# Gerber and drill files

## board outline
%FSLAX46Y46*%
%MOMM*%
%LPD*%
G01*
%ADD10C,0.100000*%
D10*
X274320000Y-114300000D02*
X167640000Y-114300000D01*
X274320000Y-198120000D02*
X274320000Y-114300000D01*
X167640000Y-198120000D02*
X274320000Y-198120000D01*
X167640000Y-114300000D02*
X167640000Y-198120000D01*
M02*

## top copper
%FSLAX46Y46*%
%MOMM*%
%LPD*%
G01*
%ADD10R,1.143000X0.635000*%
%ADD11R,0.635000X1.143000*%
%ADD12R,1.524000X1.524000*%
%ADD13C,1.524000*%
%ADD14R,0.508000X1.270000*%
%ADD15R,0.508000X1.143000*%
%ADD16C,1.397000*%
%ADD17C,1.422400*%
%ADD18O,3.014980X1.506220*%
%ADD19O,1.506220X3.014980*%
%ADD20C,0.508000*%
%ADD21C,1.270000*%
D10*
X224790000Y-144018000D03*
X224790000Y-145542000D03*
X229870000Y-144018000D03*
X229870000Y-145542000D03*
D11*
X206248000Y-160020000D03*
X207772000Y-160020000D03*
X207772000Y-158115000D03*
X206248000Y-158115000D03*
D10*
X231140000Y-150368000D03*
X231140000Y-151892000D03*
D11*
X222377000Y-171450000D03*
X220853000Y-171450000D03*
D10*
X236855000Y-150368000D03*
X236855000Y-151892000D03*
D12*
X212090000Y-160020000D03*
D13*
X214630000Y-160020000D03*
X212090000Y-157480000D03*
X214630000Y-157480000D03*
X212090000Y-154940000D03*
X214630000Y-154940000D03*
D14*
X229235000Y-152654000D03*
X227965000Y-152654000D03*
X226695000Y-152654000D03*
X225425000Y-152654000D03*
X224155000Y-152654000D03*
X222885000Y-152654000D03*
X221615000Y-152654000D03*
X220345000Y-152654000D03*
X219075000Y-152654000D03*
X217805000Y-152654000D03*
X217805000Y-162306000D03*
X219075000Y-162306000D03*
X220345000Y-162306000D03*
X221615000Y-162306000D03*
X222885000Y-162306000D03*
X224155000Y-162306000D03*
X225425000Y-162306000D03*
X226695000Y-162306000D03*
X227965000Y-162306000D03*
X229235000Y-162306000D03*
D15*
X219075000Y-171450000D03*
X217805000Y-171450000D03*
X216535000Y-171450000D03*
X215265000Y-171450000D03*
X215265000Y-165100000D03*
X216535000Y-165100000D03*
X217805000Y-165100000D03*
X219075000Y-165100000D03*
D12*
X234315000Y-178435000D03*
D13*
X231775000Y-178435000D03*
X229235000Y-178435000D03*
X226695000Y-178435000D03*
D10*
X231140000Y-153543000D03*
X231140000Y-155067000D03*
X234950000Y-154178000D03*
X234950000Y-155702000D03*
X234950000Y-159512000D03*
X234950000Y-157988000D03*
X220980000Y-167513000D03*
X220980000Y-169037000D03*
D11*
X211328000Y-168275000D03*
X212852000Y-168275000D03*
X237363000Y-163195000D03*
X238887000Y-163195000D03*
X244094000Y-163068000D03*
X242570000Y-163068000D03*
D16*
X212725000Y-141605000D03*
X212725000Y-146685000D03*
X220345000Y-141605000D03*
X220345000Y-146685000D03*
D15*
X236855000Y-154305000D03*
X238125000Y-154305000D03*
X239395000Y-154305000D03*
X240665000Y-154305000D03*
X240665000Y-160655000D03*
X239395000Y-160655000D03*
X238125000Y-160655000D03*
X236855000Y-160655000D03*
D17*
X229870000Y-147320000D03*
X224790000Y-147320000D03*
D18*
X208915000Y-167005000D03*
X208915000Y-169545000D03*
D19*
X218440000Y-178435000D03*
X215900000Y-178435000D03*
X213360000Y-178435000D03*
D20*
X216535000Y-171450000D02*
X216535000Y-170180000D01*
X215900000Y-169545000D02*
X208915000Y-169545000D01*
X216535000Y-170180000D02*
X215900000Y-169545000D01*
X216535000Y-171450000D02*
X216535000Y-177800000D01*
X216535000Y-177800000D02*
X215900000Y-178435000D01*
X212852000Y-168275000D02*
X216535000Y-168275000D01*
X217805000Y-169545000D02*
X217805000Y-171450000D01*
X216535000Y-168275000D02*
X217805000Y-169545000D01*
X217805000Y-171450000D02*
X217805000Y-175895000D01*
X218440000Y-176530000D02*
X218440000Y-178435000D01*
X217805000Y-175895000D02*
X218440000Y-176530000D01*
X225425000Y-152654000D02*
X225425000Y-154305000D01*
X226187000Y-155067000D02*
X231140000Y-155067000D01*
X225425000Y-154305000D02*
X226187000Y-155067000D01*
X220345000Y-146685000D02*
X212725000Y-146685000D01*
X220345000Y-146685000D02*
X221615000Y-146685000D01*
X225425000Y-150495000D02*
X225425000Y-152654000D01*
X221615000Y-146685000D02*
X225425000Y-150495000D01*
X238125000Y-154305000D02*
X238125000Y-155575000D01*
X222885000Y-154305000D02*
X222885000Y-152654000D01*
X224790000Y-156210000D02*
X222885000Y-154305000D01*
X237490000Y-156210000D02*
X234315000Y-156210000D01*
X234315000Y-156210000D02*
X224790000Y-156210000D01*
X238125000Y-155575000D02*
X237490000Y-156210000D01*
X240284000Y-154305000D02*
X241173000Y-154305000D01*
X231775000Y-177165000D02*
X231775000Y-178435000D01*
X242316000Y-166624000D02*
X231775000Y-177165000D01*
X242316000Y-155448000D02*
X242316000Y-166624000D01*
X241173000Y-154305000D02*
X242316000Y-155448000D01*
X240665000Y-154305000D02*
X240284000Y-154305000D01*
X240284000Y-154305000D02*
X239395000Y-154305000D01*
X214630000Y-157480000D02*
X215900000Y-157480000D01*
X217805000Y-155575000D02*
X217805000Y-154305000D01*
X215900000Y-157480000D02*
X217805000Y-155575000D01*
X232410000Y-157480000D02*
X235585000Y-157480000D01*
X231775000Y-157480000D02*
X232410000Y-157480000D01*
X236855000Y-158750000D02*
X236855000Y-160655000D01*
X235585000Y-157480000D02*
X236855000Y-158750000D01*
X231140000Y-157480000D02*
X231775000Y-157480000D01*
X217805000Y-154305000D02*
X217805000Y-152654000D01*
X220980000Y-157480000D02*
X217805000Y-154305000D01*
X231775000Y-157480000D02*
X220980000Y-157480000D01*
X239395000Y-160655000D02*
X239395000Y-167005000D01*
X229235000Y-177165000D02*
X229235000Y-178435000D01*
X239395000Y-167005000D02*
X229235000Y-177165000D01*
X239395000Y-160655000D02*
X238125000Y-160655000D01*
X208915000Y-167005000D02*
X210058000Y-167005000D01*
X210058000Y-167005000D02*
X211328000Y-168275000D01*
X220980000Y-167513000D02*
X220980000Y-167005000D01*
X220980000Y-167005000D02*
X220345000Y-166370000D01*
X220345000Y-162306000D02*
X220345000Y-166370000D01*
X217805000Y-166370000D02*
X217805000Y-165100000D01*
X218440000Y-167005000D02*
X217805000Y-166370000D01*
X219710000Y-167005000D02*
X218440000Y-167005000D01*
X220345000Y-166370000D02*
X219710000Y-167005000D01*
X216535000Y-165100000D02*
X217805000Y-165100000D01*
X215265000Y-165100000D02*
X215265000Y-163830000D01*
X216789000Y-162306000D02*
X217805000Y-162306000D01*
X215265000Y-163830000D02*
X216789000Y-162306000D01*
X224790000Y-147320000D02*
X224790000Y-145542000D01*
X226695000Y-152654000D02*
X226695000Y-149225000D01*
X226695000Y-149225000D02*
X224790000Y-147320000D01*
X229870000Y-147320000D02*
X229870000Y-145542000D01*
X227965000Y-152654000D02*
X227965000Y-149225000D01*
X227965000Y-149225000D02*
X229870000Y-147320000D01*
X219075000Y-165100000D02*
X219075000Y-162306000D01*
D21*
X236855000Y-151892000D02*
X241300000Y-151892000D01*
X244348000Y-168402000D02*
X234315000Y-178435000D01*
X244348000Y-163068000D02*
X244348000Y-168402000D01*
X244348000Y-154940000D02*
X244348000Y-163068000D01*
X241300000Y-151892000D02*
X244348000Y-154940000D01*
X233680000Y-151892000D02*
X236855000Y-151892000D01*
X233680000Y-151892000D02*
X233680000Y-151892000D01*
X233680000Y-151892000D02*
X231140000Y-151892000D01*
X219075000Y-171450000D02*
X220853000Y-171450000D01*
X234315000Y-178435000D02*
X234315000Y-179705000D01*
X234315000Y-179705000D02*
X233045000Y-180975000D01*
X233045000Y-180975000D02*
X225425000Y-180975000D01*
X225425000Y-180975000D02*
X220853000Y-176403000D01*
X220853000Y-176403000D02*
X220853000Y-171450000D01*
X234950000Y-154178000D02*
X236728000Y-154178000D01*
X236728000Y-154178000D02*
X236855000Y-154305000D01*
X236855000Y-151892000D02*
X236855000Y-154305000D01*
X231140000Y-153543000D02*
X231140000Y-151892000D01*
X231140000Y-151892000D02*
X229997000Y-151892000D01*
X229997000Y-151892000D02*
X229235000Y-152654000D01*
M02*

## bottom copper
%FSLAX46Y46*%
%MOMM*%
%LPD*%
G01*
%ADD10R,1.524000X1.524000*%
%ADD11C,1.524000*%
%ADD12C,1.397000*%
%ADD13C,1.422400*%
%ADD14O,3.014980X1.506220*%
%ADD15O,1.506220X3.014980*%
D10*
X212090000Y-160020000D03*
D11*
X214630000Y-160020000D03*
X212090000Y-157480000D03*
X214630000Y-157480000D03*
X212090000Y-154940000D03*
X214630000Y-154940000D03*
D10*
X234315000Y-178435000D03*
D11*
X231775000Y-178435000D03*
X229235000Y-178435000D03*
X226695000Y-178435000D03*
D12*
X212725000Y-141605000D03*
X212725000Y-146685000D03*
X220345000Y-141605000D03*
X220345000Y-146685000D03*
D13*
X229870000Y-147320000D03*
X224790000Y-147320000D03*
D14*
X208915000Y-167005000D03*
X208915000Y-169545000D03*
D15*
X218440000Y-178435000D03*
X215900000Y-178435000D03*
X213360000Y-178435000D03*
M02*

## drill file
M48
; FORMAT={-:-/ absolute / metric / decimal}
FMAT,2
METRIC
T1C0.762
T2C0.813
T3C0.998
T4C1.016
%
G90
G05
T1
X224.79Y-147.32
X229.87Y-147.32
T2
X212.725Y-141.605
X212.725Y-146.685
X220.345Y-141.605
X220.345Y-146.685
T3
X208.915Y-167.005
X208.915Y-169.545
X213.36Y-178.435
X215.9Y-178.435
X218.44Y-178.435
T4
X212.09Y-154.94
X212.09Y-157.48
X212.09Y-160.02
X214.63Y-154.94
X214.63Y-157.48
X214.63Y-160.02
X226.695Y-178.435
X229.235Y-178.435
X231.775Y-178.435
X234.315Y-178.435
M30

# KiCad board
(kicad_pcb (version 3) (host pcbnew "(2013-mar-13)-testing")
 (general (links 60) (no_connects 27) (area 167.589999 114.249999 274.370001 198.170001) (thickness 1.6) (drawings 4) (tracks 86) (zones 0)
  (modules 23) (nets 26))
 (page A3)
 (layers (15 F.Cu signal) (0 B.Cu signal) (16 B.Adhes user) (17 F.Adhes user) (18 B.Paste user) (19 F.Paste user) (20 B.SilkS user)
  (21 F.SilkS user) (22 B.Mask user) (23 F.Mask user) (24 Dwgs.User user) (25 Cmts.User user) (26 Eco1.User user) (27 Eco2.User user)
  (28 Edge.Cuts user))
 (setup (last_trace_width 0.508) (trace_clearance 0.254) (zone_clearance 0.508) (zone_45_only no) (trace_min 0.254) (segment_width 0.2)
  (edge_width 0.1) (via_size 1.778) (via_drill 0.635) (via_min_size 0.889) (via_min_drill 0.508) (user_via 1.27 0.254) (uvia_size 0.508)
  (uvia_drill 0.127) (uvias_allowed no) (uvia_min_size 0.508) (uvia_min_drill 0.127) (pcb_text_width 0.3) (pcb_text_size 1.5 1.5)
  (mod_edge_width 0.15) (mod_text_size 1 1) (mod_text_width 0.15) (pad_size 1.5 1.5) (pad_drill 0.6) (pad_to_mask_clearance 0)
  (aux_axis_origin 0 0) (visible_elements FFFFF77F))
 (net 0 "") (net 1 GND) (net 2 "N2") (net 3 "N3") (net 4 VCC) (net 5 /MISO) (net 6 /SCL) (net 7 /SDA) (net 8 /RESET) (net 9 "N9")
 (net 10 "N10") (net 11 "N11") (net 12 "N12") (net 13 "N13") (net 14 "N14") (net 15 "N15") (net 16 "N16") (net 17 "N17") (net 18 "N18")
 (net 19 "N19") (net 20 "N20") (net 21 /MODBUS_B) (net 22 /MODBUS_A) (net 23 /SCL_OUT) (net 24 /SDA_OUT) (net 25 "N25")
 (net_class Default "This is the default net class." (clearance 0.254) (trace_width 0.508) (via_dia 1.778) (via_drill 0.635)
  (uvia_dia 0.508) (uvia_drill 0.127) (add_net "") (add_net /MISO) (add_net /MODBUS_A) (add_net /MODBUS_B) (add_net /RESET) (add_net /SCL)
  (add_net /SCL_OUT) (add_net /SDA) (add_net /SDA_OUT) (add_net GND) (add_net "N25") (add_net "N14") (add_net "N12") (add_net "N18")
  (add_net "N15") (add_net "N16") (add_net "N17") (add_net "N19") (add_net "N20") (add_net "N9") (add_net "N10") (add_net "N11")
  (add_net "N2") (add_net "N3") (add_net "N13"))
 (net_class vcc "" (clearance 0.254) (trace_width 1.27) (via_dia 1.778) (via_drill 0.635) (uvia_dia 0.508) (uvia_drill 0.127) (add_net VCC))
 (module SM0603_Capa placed (layer F.Cu) (at 224.79 144.78 270)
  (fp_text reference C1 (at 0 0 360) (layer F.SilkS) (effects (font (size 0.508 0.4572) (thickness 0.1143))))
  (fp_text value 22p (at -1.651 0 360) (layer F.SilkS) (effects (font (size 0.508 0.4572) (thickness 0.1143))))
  (pad 1 smd rect (at -0.762 0 270) (size 0.635 1.143) (layers F.Cu F.Paste F.Mask) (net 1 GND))
  (pad 2 smd rect (at 0.762 0 270) (size 0.635 1.143) (layers F.Cu F.Paste F.Mask) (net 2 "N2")))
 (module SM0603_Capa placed (layer F.Cu) (at 229.87 144.78 270)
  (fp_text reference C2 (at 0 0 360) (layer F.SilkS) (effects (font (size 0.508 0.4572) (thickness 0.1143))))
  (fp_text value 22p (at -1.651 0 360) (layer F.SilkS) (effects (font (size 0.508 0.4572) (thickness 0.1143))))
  (pad 1 smd rect (at -0.762 0 270) (size 0.635 1.143) (layers F.Cu F.Paste F.Mask) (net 1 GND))
  (pad 2 smd rect (at 0.762 0 270) (size 0.635 1.143) (layers F.Cu F.Paste F.Mask) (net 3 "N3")))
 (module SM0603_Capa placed (layer F.Cu) (at 207.01 160.02)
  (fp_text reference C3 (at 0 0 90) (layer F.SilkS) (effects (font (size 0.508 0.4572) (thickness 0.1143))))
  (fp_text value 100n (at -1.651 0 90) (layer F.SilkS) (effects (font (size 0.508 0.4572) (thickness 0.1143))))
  (pad 1 smd rect (at -0.762 0) (size 0.635 1.143) (layers F.Cu F.Paste F.Mask) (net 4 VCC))
  (pad 2 smd rect (at 0.762 0) (size 0.635 1.143) (layers F.Cu F.Paste F.Mask) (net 1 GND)))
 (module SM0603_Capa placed (layer F.Cu) (at 207.01 158.115 180)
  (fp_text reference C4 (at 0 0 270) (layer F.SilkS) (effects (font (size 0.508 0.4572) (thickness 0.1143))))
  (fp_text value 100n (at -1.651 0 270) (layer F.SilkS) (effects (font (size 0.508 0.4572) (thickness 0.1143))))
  (pad 1 smd rect (at -0.762 0 180) (size 0.635 1.143) (layers F.Cu F.Paste F.Mask) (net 1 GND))
  (pad 2 smd rect (at 0.762 0 180) (size 0.635 1.143) (layers F.Cu F.Paste F.Mask) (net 4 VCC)))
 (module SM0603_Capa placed (layer F.Cu) (at 231.14 151.13 270)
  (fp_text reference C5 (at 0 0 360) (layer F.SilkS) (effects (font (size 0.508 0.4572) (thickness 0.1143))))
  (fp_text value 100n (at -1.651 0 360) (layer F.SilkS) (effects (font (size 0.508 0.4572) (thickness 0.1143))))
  (pad 1 smd rect (at -0.762 0 270) (size 0.635 1.143) (layers F.Cu F.Paste F.Mask) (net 1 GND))
  (pad 2 smd rect (at 0.762 0 270) (size 0.635 1.143) (layers F.Cu F.Paste F.Mask) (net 4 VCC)))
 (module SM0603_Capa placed (layer F.Cu) (at 221.615 171.45 180)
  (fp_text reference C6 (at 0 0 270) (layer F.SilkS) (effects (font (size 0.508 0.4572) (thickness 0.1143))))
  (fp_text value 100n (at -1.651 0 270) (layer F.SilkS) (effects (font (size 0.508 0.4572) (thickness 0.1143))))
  (pad 1 smd rect (at -0.762 0 180) (size 0.635 1.143) (layers F.Cu F.Paste F.Mask) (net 1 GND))
  (pad 2 smd rect (at 0.762 0 180) (size 0.635 1.143) (layers F.Cu F.Paste F.Mask) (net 4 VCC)))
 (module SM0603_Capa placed (layer F.Cu) (at 236.855 151.13 270)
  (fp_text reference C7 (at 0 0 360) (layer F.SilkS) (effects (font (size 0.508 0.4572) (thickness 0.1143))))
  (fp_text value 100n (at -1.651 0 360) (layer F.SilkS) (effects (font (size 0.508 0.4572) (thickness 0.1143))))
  (pad 1 smd rect (at -0.762 0 270) (size 0.635 1.143) (layers F.Cu F.Paste F.Mask) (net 1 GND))
  (pad 2 smd rect (at 0.762 0 270) (size 0.635 1.143) (layers F.Cu F.Paste F.Mask) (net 4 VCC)))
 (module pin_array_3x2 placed (layer B.Cu) (at 213.36 157.48 90)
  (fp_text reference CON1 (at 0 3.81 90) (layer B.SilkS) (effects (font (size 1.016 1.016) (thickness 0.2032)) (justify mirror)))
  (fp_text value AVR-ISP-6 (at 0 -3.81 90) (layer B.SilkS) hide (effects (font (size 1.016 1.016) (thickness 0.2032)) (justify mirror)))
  (pad 1 thru_hole rect (at -2.54 -1.27 90) (size 1.524 1.524) (drill 1.016) (layers *.Cu *.Mask B.SilkS) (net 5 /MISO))
  (pad 2 thru_hole circle (at -2.54 1.27 90) (size 1.524 1.524) (drill 1.016) (layers *.Cu *.Mask B.SilkS) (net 4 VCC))
  (pad 3 thru_hole circle (at 0 -1.27 90) (size 1.524 1.524) (drill 1.016) (layers *.Cu *.Mask B.SilkS) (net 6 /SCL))
  (pad 4 thru_hole circle (at 0 1.27 90) (size 1.524 1.524) (drill 1.016) (layers *.Cu *.Mask B.SilkS) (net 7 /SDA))
  (pad 5 thru_hole circle (at 2.54 -1.27 90) (size 1.524 1.524) (drill 1.016) (layers *.Cu *.Mask B.SilkS) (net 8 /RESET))
  (pad 6 thru_hole circle (at 2.54 1.27 90) (size 1.524 1.524) (drill 1.016) (layers *.Cu *.Mask B.SilkS) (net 1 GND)))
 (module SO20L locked (layer F.Cu) (at 223.52 157.48)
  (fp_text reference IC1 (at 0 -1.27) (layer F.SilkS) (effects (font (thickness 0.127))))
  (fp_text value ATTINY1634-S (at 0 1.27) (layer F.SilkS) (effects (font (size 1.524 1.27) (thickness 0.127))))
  (pad 11 smd rect (at 5.715 -4.826) (size 0.508 1.27) (layers F.Cu F.Paste F.Mask) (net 4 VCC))
  (pad 12 smd rect (at 4.445 -4.826) (size 0.508 1.27) (layers F.Cu F.Paste F.Mask) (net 3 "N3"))
  (pad 13 smd rect (at 3.175 -4.826) (size 0.508 1.27) (layers F.Cu F.Paste F.Mask) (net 2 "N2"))
  (pad 14 smd rect (at 1.905 -4.826) (size 0.508 1.27) (layers F.Cu F.Paste F.Mask) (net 8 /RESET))
  (pad 15 smd rect (at 0.635 -4.826) (size 0.508 1.27) (layers F.Cu F.Paste F.Mask) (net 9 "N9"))
  (pad 16 smd rect (at -0.635 -4.826) (size 0.508 1.27) (layers F.Cu F.Paste F.Mask) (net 6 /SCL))
  (pad 17 smd rect (at -1.905 -4.826) (size 0.508 1.27) (layers F.Cu F.Paste F.Mask) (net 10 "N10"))
  (pad 18 smd rect (at -3.175 -4.826) (size 0.508 1.27) (layers F.Cu F.Paste F.Mask) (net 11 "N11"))
  (pad 19 smd rect (at -4.445 -4.826) (size 0.508 1.27) (layers F.Cu F.Paste F.Mask) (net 5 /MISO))
  (pad 20 smd rect (at -5.715 -4.826) (size 0.508 1.27) (layers F.Cu F.Paste F.Mask) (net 7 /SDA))
  (pad 1 smd rect (at -5.715 4.826) (size 0.508 1.27) (layers F.Cu F.Paste F.Mask) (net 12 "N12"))
  (pad 2 smd rect (at -4.445 4.826) (size 0.508 1.27) (layers F.Cu F.Paste F.Mask) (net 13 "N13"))
  (pad 3 smd rect (at -3.175 4.826) (size 0.508 1.27) (layers F.Cu F.Paste F.Mask) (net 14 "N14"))
  (pad 4 smd rect (at -1.905 4.826) (size 0.508 1.27) (layers F.Cu F.Paste F.Mask) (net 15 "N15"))
  (pad 5 smd rect (at -0.635 4.826) (size 0.508 1.27) (layers F.Cu F.Paste F.Mask) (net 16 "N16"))
  (pad 6 smd rect (at 0.635 4.826) (size 0.508 1.27) (layers F.Cu F.Paste F.Mask) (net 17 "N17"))
  (pad 7 smd rect (at 1.905 4.826) (size 0.508 1.27) (layers F.Cu F.Paste F.Mask) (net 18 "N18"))
  (pad 8 smd rect (at 3.175 4.826) (size 0.508 1.27) (layers F.Cu F.Paste F.Mask) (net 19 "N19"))
  (pad 9 smd rect (at 4.445 4.826) (size 0.508 1.27) (layers F.Cu F.Paste F.Mask) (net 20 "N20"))
  (pad 10 smd rect (at 5.715 4.826) (size 0.508 1.27) (layers F.Cu F.Paste F.Mask) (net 1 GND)))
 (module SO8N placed (layer F.Cu) (at 217.17 168.275 180)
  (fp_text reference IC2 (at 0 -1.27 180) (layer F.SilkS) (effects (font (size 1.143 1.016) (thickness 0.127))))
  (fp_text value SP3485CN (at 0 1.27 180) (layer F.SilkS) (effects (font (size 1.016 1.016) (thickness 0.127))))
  (pad 8 smd rect (at -1.905 -3.175 180) (size 0.508 1.143) (layers F.Cu F.Paste F.Mask) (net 4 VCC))
  (pad 7 smd rect (at -0.635 -3.175 180) (size 0.508 1.143) (layers F.Cu F.Paste F.Mask) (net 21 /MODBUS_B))
  (pad 6 smd rect (at 0.635 -3.175 180) (size 0.508 1.143) (layers F.Cu F.Paste F.Mask) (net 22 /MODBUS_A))
  (pad 5 smd rect (at 1.905 -3.175 180) (size 0.508 1.143) (layers F.Cu F.Paste F.Mask) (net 1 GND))
  (pad 4 smd rect (at 1.905 3.175 180) (size 0.508 1.143) (layers F.Cu F.Paste F.Mask) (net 12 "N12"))
  (pad 3 smd rect (at 0.635 3.175 180) (size 0.508 1.143) (layers F.Cu F.Paste F.Mask) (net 14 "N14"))
  (pad 2 smd rect (at -0.635 3.175 180) (size 0.508 1.143) (layers F.Cu F.Paste F.Mask) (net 14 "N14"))
  (pad 1 smd rect (at -1.905 3.175 180) (size 0.508 1.143) (layers F.Cu F.Paste F.Mask) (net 13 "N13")))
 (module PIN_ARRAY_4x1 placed (layer B.Cu) (at 230.505 178.435 180)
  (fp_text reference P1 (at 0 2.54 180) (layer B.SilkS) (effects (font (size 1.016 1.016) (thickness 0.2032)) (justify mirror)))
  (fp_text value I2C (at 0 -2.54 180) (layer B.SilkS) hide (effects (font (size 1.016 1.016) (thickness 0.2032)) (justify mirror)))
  (pad 1 thru_hole rect (at -3.81 0 180) (size 1.524 1.524) (drill 1.016) (layers *.Cu *.Mask B.SilkS) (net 4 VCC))
  (pad 2 thru_hole circle (at -1.27 0 180) (size 1.524 1.524) (drill 1.016) (layers *.Cu *.Mask B.SilkS) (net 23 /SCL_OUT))
  (pad 3 thru_hole circle (at 1.27 0 180) (size 1.524 1.524) (drill 1.016) (layers *.Cu *.Mask B.SilkS) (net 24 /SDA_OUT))
  (pad 4 thru_hole circle (at 3.81 0 180) (size 1.524 1.524) (drill 1.016) (layers *.Cu *.Mask B.SilkS) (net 1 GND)))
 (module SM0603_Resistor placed (layer F.Cu) (at 231.14 154.305 270)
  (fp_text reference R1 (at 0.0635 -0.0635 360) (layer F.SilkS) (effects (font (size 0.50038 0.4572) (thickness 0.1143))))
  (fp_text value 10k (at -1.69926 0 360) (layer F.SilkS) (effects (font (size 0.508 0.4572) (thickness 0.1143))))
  (pad 1 smd rect (at -0.762 0 270) (size 0.635 1.143) (layers F.Cu F.Paste F.Mask) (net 4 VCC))
  (pad 2 smd rect (at 0.762 0 270) (size 0.635 1.143) (layers F.Cu F.Paste F.Mask) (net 8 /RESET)))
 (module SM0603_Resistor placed (layer F.Cu) (at 234.95 154.94 270)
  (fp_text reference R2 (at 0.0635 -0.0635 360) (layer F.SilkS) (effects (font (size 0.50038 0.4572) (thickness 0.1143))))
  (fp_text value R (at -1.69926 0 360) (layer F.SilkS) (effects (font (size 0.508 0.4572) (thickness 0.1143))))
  (pad 1 smd rect (at -0.762 0 270) (size 0.635 1.143) (layers F.Cu F.Paste F.Mask) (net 4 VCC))
  (pad 2 smd rect (at 0.762 0 270) (size 0.635 1.143) (layers F.Cu F.Paste F.Mask) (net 6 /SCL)))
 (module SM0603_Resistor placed (layer F.Cu) (at 234.95 158.75 90)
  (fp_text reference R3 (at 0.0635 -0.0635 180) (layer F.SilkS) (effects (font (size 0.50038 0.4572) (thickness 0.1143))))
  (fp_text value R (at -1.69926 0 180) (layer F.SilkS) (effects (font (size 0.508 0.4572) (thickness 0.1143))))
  (pad 1 smd rect (at -0.762 0 90) (size 0.635 1.143) (layers F.Cu F.Paste F.Mask) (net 4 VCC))
  (pad 2 smd rect (at 0.762 0 90) (size 0.635 1.143) (layers F.Cu F.Paste F.Mask) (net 7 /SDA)))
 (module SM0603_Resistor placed (layer F.Cu) (at 220.98 168.275 270)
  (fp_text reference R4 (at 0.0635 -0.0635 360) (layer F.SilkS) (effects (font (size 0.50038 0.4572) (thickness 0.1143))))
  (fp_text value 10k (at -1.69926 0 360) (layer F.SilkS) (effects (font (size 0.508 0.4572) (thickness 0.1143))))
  (pad 1 smd rect (at -0.762 0 270) (size 0.635 1.143) (layers F.Cu F.Paste F.Mask) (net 14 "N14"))
  (pad 2 smd rect (at 0.762 0 270) (size 0.635 1.143) (layers F.Cu F.Paste F.Mask) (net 1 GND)))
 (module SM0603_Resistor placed (layer F.Cu) (at 212.09 168.275)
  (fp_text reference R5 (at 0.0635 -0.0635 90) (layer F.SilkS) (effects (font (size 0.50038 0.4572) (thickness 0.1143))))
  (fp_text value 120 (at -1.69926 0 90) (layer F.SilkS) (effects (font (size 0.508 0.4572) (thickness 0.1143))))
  (pad 1 smd rect (at -0.762 0) (size 0.635 1.143) (layers F.Cu F.Paste F.Mask) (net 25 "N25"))
  (pad 2 smd rect (at 0.762 0) (size 0.635 1.143) (layers F.Cu F.Paste F.Mask) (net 21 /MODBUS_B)))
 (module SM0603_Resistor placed (layer F.Cu) (at 238.125 163.195)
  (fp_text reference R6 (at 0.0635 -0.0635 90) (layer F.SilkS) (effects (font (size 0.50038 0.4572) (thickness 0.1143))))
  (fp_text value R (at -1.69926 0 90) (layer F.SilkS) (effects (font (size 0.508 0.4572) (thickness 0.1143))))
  (pad 1 smd rect (at -0.762 0) (size 0.635 1.143) (layers F.Cu F.Paste F.Mask) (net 4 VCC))
  (pad 2 smd rect (at 0.762 0) (size 0.635 1.143) (layers F.Cu F.Paste F.Mask) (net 24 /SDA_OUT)))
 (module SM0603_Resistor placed (layer F.Cu) (at 243.332 163.068 180)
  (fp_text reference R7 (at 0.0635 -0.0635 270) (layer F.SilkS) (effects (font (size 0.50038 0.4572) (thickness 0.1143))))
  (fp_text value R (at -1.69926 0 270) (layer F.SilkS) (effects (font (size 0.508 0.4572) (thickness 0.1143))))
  (pad 1 smd rect (at -0.762 0 180) (size 0.635 1.143) (layers F.Cu F.Paste F.Mask) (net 4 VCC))
  (pad 2 smd rect (at 0.762 0 180) (size 0.635 1.143) (layers F.Cu F.Paste F.Mask) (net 23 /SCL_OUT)))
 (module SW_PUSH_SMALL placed (layer B.Cu) (at 216.535 144.145 180)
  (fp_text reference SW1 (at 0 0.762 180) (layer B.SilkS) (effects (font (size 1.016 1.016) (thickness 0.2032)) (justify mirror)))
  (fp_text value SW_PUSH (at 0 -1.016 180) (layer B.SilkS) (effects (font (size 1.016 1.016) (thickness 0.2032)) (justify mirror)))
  (pad 1 thru_hole circle (at 3.81 2.54 180) (size 1.397 1.397) (drill 0.8128) (layers *.Cu *.Mask B.SilkS) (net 1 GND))
  (pad 2 thru_hole circle (at 3.81 -2.54 180) (size 1.397 1.397) (drill 0.8128) (layers *.Cu *.Mask B.SilkS) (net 8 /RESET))
  (pad 1 thru_hole circle (at -3.81 2.54 180) (size 1.397 1.397) (drill 0.8128) (layers *.Cu *.Mask B.SilkS) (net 1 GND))
  (pad 2 thru_hole circle (at -3.81 -2.54 180) (size 1.397 1.397) (drill 0.8128) (layers *.Cu *.Mask B.SilkS) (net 8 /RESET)))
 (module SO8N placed (layer F.Cu) (at 238.76 157.48)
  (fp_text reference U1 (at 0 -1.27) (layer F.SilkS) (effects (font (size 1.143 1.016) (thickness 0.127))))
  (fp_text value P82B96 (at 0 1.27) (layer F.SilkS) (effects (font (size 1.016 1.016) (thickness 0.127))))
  (pad 8 smd rect (at -1.905 -3.175) (size 0.508 1.143) (layers F.Cu F.Paste F.Mask) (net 4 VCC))
  (pad 7 smd rect (at -0.635 -3.175) (size 0.508 1.143) (layers F.Cu F.Paste F.Mask) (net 6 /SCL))
  (pad 6 smd rect (at 0.635 -3.175) (size 0.508 1.143) (layers F.Cu F.Paste F.Mask) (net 23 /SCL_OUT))
  (pad 5 smd rect (at 1.905 -3.175) (size 0.508 1.143) (layers F.Cu F.Paste F.Mask) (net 23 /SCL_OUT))
  (pad 4 smd rect (at 1.905 3.175) (size 0.508 1.143) (layers F.Cu F.Paste F.Mask) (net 1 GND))
  (pad 3 smd rect (at 0.635 3.175) (size 0.508 1.143) (layers F.Cu F.Paste F.Mask) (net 24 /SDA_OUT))
  (pad 2 smd rect (at -0.635 3.175) (size 0.508 1.143) (layers F.Cu F.Paste F.Mask) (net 24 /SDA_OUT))
  (pad 1 smd rect (at -1.905 3.175) (size 0.508 1.143) (layers F.Cu F.Paste F.Mask) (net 7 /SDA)))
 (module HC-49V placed (layer B.Cu) (at 227.33 147.32 180) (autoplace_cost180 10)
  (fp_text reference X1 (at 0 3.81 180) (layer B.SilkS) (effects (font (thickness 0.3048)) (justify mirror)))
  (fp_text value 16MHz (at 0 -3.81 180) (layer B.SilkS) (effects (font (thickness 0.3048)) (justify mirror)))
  (pad 1 thru_hole circle (at -2.54 0 180) (size 1.4224 1.4224) (drill 0.762) (layers *.Cu *.Mask B.SilkS) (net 3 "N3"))
  (pad 2 thru_hole circle (at 2.54 0 180) (size 1.4224 1.4224) (drill 0.762) (layers *.Cu *.Mask B.SilkS) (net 2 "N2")))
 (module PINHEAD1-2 (layer B.Cu) (at 208.915 168.275 270)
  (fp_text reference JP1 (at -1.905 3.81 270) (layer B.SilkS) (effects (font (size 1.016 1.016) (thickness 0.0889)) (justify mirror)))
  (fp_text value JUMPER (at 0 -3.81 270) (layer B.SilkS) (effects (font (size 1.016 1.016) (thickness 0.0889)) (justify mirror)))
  (pad 1 thru_hole oval (at -1.27 0 270) (size 1.50622 3.01498) (drill 0.99822) (layers *.Cu B.Paste B.SilkS B.Mask) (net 25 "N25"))
  (pad 2 thru_hole oval (at 1.27 0 270) (size 1.50622 3.01498) (drill 0.99822) (layers *.Cu B.Paste B.SilkS B.Mask) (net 22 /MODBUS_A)))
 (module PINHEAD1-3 (layer B.Cu) (at 215.9 178.435 180)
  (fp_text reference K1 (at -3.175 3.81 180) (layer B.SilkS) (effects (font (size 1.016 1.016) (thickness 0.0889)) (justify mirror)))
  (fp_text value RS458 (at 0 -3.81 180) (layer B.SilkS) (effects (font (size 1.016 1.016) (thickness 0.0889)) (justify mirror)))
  (pad 1 thru_hole oval (at -2.54 0 180) (size 1.50622 3.01498) (drill 0.99822) (layers *.Cu B.Paste B.SilkS B.Mask) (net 21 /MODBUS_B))
  (pad 2 thru_hole oval (at 0 0 180) (size 1.50622 3.01498) (drill 0.99822) (layers *.Cu B.Paste B.SilkS B.Mask) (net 22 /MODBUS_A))
  (pad 3 thru_hole oval (at 2.54 0 180) (size 1.50622 3.01498) (drill 0.99822) (layers *.Cu B.Paste B.SilkS B.Mask) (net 1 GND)))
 (gr_line (start 274.32 114.3) (end 167.64 114.3) (angle 90) (layer Edge.Cuts) (width 0.1))
 (gr_line (start 274.32 198.12) (end 274.32 114.3) (angle 90) (layer Edge.Cuts) (width 0.1))
 (gr_line (start 167.64 198.12) (end 274.32 198.12) (angle 90) (layer Edge.Cuts) (width 0.1))
 (gr_line (start 167.64 114.3) (end 167.64 198.12) (angle 90) (layer Edge.Cuts) (width 0.1))
 (segment (start 216.535 171.45) (end 216.535 170.18) (width 0.508) (layer F.Cu) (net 22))
 (segment (start 215.9 169.545) (end 208.915 169.545) (width 0.508) (layer F.Cu) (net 22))
 (segment (start 216.535 170.18) (end 215.9 169.545) (width 0.508) (layer F.Cu) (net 22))
 (segment (start 216.535 171.45) (end 216.535 177.8) (width 0.508) (layer F.Cu) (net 22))
 (segment (start 216.535 177.8) (end 215.9 178.435) (width 0.508) (layer F.Cu) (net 22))
 (segment (start 212.852 168.275) (end 216.535 168.275) (width 0.508) (layer F.Cu) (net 21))
 (segment (start 217.805 169.545) (end 217.805 171.45) (width 0.508) (layer F.Cu) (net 21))
 (segment (start 216.535 168.275) (end 217.805 169.545) (width 0.508) (layer F.Cu) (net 21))
 (segment (start 217.805 171.45) (end 217.805 175.895) (width 0.508) (layer F.Cu) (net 21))
 (segment (start 218.44 176.53) (end 218.44 178.435) (width 0.508) (layer F.Cu) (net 21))
 (segment (start 217.805 175.895) (end 218.44 176.53) (width 0.508) (layer F.Cu) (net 21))
 (segment (start 225.425 152.654) (end 225.425 154.305) (width 0.508) (layer F.Cu) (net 8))
 (segment (start 226.187 155.067) (end 231.14 155.067) (width 0.508) (layer F.Cu) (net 8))
 (segment (start 225.425 154.305) (end 226.187 155.067) (width 0.508) (layer F.Cu) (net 8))
 (segment (start 220.345 146.685) (end 212.725 146.685) (width 0.508) (layer F.Cu) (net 8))
 (segment (start 220.345 146.685) (end 221.615 146.685) (width 0.508) (layer F.Cu) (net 8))
 (segment (start 225.425 150.495) (end 225.425 152.654) (width 0.508) (layer F.Cu) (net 8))
 (segment (start 221.615 146.685) (end 225.425 150.495) (width 0.508) (layer F.Cu) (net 8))
 (segment (start 238.125 154.305) (end 238.125 155.575) (width 0.508) (layer F.Cu) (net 6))
 (segment (start 222.885 154.305) (end 222.885 152.654) (width 0.508) (layer F.Cu) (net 6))
 (segment (start 224.79 156.21) (end 222.885 154.305) (width 0.508) (layer F.Cu) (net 6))
 (segment (start 237.49 156.21) (end 234.315 156.21) (width 0.508) (layer F.Cu) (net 6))
 (segment (start 234.315 156.21) (end 224.79 156.21) (width 0.508) (layer F.Cu) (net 6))
 (segment (start 238.125 155.575) (end 237.49 156.21) (width 0.508) (layer F.Cu) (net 6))
 (segment (start 240.284 154.305) (end 241.173 154.305) (width 0.508) (layer F.Cu) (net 23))
 (segment (start 231.775 177.165) (end 231.775 178.435) (width 0.508) (layer F.Cu) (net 23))
 (segment (start 242.316 166.624) (end 231.775 177.165) (width 0.508) (layer F.Cu) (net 23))
 (segment (start 242.316 155.448) (end 242.316 166.624) (width 0.508) (layer F.Cu) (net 23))
 (segment (start 241.173 154.305) (end 242.316 155.448) (width 0.508) (layer F.Cu) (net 23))
 (segment (start 240.665 154.305) (end 240.284 154.305) (width 0.508) (layer F.Cu) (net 23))
 (segment (start 240.284 154.305) (end 239.395 154.305) (width 0.508) (layer F.Cu) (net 23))
 (segment (start 214.63 157.48) (end 215.9 157.48) (width 0.508) (layer F.Cu) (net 7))
 (segment (start 217.805 155.575) (end 217.805 154.305) (width 0.508) (layer F.Cu) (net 7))
 (segment (start 215.9 157.48) (end 217.805 155.575) (width 0.508) (layer F.Cu) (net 7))
 (segment (start 232.41 157.48) (end 235.585 157.48) (width 0.508) (layer F.Cu) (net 7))
 (segment (start 231.775 157.48) (end 232.41 157.48) (width 0.508) (layer F.Cu) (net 7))
 (segment (start 236.855 158.75) (end 236.855 160.655) (width 0.508) (layer F.Cu) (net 7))
 (segment (start 235.585 157.48) (end 236.855 158.75) (width 0.508) (layer F.Cu) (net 7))
 (segment (start 231.14 157.48) (end 231.775 157.48) (width 0.508) (layer F.Cu) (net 7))
 (segment (start 217.805 154.305) (end 217.805 152.654) (width 0.508) (layer F.Cu) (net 7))
 (segment (start 220.98 157.48) (end 217.805 154.305) (width 0.508) (layer F.Cu) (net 7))
 (segment (start 231.775 157.48) (end 220.98 157.48) (width 0.508) (layer F.Cu) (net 7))
 (segment (start 239.395 160.655) (end 239.395 167.005) (width 0.508) (layer F.Cu) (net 24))
 (segment (start 229.235 177.165) (end 229.235 178.435) (width 0.508) (layer F.Cu) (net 24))
 (segment (start 239.395 167.005) (end 229.235 177.165) (width 0.508) (layer F.Cu) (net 24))
 (segment (start 239.395 160.655) (end 238.125 160.655) (width 0.508) (layer F.Cu) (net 24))
 (segment (start 208.915 167.005) (end 210.058 167.005) (width 0.508) (layer F.Cu) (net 25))
 (segment (start 210.058 167.005) (end 211.328 168.275) (width 0.508) (layer F.Cu) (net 25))
 (segment (start 220.98 167.513) (end 220.98 167.005) (width 0.508) (layer F.Cu) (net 14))
 (segment (start 220.98 167.005) (end 220.345 166.37) (width 0.508) (layer F.Cu) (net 14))
 (segment (start 220.345 162.306) (end 220.345 166.37) (width 0.508) (layer F.Cu) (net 14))
 (segment (start 217.805 166.37) (end 217.805 165.1) (width 0.508) (layer F.Cu) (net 14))
 (segment (start 218.44 167.005) (end 217.805 166.37) (width 0.508) (layer F.Cu) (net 14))
 (segment (start 219.71 167.005) (end 218.44 167.005) (width 0.508) (layer F.Cu) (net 14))
 (segment (start 220.345 166.37) (end 219.71 167.005) (width 0.508) (layer F.Cu) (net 14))
 (segment (start 216.535 165.1) (end 217.805 165.1) (width 0.508) (layer F.Cu) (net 14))
 (segment (start 215.265 165.1) (end 215.265 163.83) (width 0.508) (layer F.Cu) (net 12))
 (segment (start 216.789 162.306) (end 217.805 162.306) (width 0.508) (layer F.Cu) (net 12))
 (segment (start 215.265 163.83) (end 216.789 162.306) (width 0.508) (layer F.Cu) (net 12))
 (segment (start 224.79 147.32) (end 224.79 145.542) (width 0.508) (layer F.Cu) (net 2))
 (segment (start 226.695 152.654) (end 226.695 149.225) (width 0.508) (layer F.Cu) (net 2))
 (segment (start 226.695 149.225) (end 224.79 147.32) (width 0.508) (layer F.Cu) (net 2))
 (segment (start 229.87 147.32) (end 229.87 145.542) (width 0.508) (layer F.Cu) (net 3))
 (segment (start 227.965 152.654) (end 227.965 149.225) (width 0.508) (layer F.Cu) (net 3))
 (segment (start 227.965 149.225) (end 229.87 147.32) (width 0.508) (layer F.Cu) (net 3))
 (segment (start 219.075 165.1) (end 219.075 162.306) (width 0.508) (layer F.Cu) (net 13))
 (segment (start 236.855 151.892) (end 241.3 151.892) (width 1.27) (layer F.Cu) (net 4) (status 400000))
 (segment (start 244.348 168.402) (end 234.315 178.435) (width 1.27) (layer F.Cu) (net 4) (status 800000))
 (segment (start 244.348 163.068) (end 244.348 168.402) (width 1.27) (layer F.Cu) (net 4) (status 400000))
 (segment (start 244.348 154.94) (end 244.348 163.068) (width 1.27) (layer F.Cu) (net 4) (status 800000))
 (segment (start 241.3 151.892) (end 244.348 154.94) (width 1.27) (layer F.Cu) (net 4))
 (segment (start 233.68 151.892) (end 236.855 151.892) (width 1.27) (layer F.Cu) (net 4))
 (segment (start 233.68 151.892) (end 233.68 151.892) (width 1.27) (layer F.Cu) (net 4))
 (segment (start 233.68 151.892) (end 231.14 151.892) (width 1.27) (layer F.Cu) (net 4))
 (segment (start 219.075 171.45) (end 220.853 171.45) (width 1.27) (layer F.Cu) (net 4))
 (segment (start 234.315 178.435) (end 234.315 179.705) (width 1.27) (layer F.Cu) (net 4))
 (segment (start 234.315 179.705) (end 233.045 180.975) (width 1.27) (layer F.Cu) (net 4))
 (segment (start 233.045 180.975) (end 225.425 180.975) (width 1.27) (layer F.Cu) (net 4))
 (segment (start 225.425 180.975) (end 220.853 176.403) (width 1.27) (layer F.Cu) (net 4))
 (segment (start 220.853 176.403) (end 220.853 171.45) (width 1.27) (layer F.Cu) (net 4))
 (segment (start 234.95 154.178) (end 236.728 154.178) (width 1.27) (layer F.Cu) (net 4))
 (segment (start 236.728 154.178) (end 236.855 154.305) (width 1.27) (layer F.Cu) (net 4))
 (segment (start 236.855 151.892) (end 236.855 154.305) (width 1.27) (layer F.Cu) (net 4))
 (segment (start 231.14 153.543) (end 231.14 151.892) (width 1.27) (layer F.Cu) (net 4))
 (segment (start 231.14 151.892) (end 229.997 151.892) (width 1.27) (layer F.Cu) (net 4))
 (segment (start 229.997 151.892) (end 229.235 152.654) (width 1.27) (layer F.Cu) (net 4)))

